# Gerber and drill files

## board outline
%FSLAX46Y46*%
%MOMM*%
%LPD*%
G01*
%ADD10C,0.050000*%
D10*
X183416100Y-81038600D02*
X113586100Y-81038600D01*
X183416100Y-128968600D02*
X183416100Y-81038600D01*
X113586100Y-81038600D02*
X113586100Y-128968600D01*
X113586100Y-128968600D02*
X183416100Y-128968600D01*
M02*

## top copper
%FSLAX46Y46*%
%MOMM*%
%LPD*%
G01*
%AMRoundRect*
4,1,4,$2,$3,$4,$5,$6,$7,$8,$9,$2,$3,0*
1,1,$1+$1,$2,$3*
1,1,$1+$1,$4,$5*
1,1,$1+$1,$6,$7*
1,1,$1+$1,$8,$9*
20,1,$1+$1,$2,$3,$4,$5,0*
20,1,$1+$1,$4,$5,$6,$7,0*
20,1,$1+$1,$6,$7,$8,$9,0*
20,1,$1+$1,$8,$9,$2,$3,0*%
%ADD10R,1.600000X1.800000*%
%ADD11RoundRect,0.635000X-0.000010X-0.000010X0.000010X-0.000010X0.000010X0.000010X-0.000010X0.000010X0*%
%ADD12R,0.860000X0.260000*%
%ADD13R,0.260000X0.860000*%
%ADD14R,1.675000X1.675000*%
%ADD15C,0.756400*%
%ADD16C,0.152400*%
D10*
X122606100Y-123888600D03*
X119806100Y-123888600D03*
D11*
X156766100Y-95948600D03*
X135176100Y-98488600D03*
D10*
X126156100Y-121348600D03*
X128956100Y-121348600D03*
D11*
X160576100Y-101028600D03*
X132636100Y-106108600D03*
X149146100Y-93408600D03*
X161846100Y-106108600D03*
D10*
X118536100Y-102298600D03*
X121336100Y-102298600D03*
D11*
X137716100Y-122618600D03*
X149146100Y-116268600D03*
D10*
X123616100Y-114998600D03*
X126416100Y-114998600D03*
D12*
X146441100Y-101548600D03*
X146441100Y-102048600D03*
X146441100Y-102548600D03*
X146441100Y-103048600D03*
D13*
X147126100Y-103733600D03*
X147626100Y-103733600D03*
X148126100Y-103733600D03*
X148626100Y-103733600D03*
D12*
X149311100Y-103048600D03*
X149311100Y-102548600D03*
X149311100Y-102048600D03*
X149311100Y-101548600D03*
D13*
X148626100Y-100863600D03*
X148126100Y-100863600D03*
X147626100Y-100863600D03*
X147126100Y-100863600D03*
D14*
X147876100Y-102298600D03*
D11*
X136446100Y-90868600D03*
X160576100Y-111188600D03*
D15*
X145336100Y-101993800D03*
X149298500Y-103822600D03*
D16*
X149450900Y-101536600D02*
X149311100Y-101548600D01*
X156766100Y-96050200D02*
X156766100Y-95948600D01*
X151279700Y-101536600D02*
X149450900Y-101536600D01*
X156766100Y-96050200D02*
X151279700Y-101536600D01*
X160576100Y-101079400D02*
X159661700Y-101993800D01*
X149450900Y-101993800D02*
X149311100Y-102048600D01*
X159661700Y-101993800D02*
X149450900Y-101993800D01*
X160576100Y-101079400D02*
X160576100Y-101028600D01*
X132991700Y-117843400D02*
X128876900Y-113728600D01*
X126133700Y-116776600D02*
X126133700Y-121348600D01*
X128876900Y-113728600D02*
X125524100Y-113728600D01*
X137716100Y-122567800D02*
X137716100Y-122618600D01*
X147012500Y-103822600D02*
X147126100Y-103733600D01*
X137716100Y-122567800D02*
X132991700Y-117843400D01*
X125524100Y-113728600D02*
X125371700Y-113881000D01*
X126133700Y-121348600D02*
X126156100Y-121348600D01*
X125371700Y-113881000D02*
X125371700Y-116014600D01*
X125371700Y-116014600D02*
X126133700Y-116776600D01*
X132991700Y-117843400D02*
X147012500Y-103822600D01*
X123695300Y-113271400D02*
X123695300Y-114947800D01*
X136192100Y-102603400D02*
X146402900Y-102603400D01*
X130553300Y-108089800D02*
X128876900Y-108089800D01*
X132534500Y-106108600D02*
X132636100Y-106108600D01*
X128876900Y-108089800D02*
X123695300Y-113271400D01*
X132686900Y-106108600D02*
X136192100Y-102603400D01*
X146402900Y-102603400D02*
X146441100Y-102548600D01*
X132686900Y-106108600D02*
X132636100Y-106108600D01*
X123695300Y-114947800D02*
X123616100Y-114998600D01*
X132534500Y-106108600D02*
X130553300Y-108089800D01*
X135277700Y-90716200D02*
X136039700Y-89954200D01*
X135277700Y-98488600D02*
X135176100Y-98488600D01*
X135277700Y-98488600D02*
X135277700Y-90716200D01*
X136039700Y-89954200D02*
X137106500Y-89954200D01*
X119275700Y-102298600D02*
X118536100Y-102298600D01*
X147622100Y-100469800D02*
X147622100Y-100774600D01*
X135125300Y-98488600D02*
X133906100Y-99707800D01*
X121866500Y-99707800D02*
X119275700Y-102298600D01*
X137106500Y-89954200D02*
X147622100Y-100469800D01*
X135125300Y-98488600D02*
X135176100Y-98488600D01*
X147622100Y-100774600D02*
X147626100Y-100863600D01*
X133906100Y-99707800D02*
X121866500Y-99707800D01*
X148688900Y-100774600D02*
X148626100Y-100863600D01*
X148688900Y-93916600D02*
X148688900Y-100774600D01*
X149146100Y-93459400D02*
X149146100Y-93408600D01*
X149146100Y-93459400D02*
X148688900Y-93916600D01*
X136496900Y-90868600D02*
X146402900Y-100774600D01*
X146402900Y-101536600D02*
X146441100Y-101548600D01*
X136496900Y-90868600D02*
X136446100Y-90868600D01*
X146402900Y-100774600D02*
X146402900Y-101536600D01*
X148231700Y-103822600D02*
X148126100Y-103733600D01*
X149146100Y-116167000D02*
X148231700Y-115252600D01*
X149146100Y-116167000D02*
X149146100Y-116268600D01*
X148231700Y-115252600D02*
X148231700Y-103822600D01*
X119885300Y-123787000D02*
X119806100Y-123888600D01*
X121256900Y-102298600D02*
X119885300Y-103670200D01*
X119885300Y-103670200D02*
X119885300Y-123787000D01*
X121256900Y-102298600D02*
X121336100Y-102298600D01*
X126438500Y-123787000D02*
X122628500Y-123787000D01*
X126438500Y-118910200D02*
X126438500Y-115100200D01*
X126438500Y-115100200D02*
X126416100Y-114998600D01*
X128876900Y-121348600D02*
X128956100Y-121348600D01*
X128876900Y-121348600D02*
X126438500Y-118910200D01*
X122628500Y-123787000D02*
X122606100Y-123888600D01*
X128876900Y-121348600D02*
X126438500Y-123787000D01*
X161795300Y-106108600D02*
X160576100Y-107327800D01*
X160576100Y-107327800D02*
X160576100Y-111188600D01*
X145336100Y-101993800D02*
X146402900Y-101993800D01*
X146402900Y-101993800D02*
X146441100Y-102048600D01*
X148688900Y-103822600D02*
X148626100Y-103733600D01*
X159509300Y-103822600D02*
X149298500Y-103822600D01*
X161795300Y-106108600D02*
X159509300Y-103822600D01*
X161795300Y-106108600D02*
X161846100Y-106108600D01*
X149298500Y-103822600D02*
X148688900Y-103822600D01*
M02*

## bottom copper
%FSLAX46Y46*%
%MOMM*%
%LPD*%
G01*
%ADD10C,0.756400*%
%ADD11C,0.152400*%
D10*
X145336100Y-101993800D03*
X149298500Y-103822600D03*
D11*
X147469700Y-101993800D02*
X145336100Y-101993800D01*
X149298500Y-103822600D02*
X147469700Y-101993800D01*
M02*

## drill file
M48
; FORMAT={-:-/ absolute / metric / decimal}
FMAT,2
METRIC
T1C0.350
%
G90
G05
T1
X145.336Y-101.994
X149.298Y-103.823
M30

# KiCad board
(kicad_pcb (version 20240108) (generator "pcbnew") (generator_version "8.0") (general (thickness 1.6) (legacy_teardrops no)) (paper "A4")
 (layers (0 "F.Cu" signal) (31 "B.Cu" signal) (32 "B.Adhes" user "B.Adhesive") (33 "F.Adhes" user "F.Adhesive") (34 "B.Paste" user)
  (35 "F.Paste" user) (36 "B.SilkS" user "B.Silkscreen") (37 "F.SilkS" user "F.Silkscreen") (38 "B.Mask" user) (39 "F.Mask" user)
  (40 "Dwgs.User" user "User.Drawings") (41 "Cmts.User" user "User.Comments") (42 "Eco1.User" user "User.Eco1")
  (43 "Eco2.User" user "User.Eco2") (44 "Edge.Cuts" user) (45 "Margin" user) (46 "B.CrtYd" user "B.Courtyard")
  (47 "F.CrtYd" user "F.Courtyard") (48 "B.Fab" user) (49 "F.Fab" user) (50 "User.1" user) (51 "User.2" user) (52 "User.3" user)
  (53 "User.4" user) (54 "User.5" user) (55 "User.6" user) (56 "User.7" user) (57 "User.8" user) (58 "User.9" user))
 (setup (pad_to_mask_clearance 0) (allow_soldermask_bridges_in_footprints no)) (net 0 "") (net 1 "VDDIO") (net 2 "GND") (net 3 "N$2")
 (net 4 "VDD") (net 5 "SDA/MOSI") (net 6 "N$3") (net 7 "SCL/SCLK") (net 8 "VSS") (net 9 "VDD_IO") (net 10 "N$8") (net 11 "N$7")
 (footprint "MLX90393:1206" (layer "F.Cu") (at 121.2061 123.8886 180)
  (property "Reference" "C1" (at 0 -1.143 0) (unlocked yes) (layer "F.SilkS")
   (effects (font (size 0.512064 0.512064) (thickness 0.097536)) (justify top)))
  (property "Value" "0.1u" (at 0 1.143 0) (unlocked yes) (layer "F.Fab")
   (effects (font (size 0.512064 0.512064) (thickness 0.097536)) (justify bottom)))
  (pad "1" smd rect (at -1.4 0 180) (size 1.6 1.8) (layers "F.Cu" "F.Paste" "F.Mask") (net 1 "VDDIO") (solder_mask_margin 0.1016)
   (thermal_bridge_angle 0))
  (pad "2" smd rect (at 1.4 0 180) (size 1.6 1.8) (layers "F.Cu" "F.Paste" "F.Mask") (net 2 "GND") (solder_mask_margin 0.1016)
   (thermal_bridge_angle 0)))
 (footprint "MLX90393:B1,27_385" (layer "F.Cu") (at 156.7661 95.9486)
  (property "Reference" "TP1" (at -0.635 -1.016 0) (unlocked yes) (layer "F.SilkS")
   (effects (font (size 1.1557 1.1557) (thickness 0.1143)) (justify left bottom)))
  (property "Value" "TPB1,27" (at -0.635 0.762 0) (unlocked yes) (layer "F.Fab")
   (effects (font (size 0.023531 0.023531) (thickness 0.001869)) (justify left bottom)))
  (pad "TP" smd roundrect (at 0 0) (size 1.27 1.27) (layers "F.Cu" "F.Mask") (roundrect_rratio 0.5) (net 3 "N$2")
   (solder_mask_margin 0.1016) (thermal_bridge_angle 0)))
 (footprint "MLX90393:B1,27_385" (layer "F.Cu") (at 135.1761 98.4886)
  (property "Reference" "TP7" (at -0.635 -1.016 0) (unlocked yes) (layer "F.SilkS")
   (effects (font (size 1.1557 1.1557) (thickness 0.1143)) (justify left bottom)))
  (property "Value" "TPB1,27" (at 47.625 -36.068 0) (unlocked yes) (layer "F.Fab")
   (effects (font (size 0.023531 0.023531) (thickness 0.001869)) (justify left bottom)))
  (pad "TP" smd roundrect (at 0 0) (size 1.27 1.27) (layers "F.Cu" "F.Mask") (roundrect_rratio 0.5) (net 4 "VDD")
   (solder_mask_margin 0.1016) (thermal_bridge_angle 0)))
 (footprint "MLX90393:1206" (layer "F.Cu") (at 127.5561 121.3486)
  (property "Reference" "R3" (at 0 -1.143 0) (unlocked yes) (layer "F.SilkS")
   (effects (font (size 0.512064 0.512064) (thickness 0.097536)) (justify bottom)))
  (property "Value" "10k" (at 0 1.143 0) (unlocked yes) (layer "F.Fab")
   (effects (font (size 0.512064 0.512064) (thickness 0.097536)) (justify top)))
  (pad "1" smd rect (at -1.4 0) (size 1.6 1.8) (layers "F.Cu" "F.Paste" "F.Mask") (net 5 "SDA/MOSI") (solder_mask_margin 0.1016)
   (thermal_bridge_angle 0))
  (pad "2" smd rect (at 1.4 0) (size 1.6 1.8) (layers "F.Cu" "F.Paste" "F.Mask") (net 1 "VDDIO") (solder_mask_margin 0.1016)
   (thermal_bridge_angle 0)))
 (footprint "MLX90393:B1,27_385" (layer "F.Cu") (at 160.5761 101.0286)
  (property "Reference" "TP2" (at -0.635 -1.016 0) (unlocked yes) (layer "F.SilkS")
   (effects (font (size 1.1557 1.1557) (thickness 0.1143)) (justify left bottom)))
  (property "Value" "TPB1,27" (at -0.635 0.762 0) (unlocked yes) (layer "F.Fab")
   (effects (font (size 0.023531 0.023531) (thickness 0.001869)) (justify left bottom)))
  (pad "TP" smd roundrect (at 0 0) (size 1.27 1.27) (layers "F.Cu" "F.Mask") (roundrect_rratio 0.5) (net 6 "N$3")
   (solder_mask_margin 0.1016) (thermal_bridge_angle 0)))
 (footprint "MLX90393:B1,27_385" (layer "F.Cu") (at 132.6361 106.1086)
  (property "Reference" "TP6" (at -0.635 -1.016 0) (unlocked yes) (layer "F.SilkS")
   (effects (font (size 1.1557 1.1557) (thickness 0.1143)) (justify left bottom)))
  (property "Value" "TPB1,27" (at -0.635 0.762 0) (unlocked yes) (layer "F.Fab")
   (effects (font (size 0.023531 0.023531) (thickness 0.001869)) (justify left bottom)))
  (pad "TP" smd roundrect (at 0 0) (size 1.27 1.27) (layers "F.Cu" "F.Mask") (roundrect_rratio 0.5) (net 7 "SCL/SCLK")
   (solder_mask_margin 0.1016) (thermal_bridge_angle 0)))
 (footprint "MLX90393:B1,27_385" (layer "F.Cu") (at 149.1461 93.4086)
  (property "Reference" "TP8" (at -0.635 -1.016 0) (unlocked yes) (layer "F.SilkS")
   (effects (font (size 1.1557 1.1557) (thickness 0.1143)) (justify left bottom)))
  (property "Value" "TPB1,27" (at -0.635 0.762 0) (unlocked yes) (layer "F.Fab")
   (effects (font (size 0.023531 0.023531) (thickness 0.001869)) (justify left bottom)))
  (pad "TP" smd roundrect (at 0 0) (size 1.27 1.27) (layers "F.Cu" "F.Mask") (roundrect_rratio 0.5) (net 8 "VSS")
   (solder_mask_margin 0.1016) (thermal_bridge_angle 0)))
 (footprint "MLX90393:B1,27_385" (layer "F.Cu") (at 161.8461 106.1086)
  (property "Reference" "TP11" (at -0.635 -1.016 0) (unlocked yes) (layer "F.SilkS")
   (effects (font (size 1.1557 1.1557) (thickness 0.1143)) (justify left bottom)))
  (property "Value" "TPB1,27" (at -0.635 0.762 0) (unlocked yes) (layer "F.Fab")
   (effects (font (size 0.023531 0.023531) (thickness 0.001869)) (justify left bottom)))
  (pad "TP" smd roundrect (at 0 0) (size 1.27 1.27) (layers "F.Cu" "F.Mask") (roundrect_rratio 0.5) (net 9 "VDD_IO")
   (solder_mask_margin 0.1016) (thermal_bridge_angle 0)))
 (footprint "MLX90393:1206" (layer "F.Cu") (at 119.9361 102.2986)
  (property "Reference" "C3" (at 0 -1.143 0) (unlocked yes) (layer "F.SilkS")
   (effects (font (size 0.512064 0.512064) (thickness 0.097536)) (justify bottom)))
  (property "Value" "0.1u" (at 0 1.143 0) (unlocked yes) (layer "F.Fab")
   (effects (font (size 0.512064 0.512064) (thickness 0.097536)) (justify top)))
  (pad "1" smd rect (at -1.4 0) (size 1.6 1.8) (layers "F.Cu" "F.Paste" "F.Mask") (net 4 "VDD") (solder_mask_margin 0.1016)
   (thermal_bridge_angle 0))
  (pad "2" smd rect (at 1.4 0) (size 1.6 1.8) (layers "F.Cu" "F.Paste" "F.Mask") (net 2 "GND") (solder_mask_margin 0.1016)
   (thermal_bridge_angle 0)))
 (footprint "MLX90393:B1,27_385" (layer "F.Cu") (at 137.7161 122.6186)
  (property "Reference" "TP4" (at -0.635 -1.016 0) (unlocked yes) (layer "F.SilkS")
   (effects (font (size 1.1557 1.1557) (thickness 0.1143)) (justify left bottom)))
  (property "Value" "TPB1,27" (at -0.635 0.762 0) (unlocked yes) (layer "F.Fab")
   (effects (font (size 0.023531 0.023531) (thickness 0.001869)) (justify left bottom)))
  (pad "TP" smd roundrect (at 0 0) (size 1.27 1.27) (layers "F.Cu" "F.Mask") (roundrect_rratio 0.5) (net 5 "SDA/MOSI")
   (solder_mask_margin 0.1016) (thermal_bridge_angle 0)))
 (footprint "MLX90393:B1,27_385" (layer "F.Cu") (at 149.1461 116.2686)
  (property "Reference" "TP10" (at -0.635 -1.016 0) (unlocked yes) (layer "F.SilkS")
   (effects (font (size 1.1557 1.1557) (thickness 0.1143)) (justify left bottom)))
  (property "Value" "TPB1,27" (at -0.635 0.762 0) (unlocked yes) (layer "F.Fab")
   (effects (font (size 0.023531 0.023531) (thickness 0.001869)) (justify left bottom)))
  (pad "TP" smd roundrect (at 0 0) (size 1.27 1.27) (layers "F.Cu" "F.Mask") (roundrect_rratio 0.5) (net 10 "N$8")
   (solder_mask_margin 0.1016) (thermal_bridge_angle 0)))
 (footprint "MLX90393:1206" (layer "F.Cu") (at 125.0161 114.9986)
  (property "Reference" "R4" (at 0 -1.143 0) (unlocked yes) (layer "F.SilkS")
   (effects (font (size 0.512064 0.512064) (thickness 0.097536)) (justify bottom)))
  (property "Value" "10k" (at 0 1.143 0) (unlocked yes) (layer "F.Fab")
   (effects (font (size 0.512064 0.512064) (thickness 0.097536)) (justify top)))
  (pad "1" smd rect (at -1.4 0) (size 1.6 1.8) (layers "F.Cu" "F.Paste" "F.Mask") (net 7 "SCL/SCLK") (solder_mask_margin 0.1016)
   (thermal_bridge_angle 0))
  (pad "2" smd rect (at 1.4 0) (size 1.6 1.8) (layers "F.Cu" "F.Paste" "F.Mask") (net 1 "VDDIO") (solder_mask_margin 0.1016)
   (thermal_bridge_angle 0)))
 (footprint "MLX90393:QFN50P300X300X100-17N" (layer "F.Cu") (at 147.8761 102.2986)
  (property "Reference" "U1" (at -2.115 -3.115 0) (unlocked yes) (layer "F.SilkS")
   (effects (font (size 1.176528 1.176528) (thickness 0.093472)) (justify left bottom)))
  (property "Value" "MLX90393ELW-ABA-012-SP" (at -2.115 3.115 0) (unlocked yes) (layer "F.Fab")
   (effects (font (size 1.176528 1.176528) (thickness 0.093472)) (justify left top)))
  (pad "1" smd rect (at -1.435 -0.75) (size 0.86 0.26) (layers "F.Cu" "F.Paste" "F.Mask") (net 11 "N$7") (solder_mask_margin 0.1016)
   (thermal_bridge_angle 0))
  (pad "2" smd rect (at -1.435 -0.25) (size 0.86 0.26) (layers "F.Cu" "F.Paste" "F.Mask") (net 9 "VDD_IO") (solder_mask_margin 0.1016)
   (thermal_bridge_angle 0))
  (pad "3" smd rect (at -1.435 0.25) (size 0.86 0.26) (layers "F.Cu" "F.Paste" "F.Mask") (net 7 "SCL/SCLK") (solder_mask_margin 0.1016)
   (thermal_bridge_angle 0))
  (pad "4" smd rect (at -1.435 0.75) (size 0.86 0.26) (layers "F.Cu" "F.Paste" "F.Mask") (solder_mask_margin 0.1016)
   (thermal_bridge_angle 0))
  (pad "5" smd rect (at -0.75 1.435) (size 0.26 0.86) (layers "F.Cu" "F.Paste" "F.Mask") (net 5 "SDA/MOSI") (solder_mask_margin 0.1016)
   (thermal_bridge_angle 0))
  (pad "6" smd rect (at -0.25 1.435) (size 0.26 0.86) (layers "F.Cu" "F.Paste" "F.Mask") (solder_mask_margin 0.1016)
   (thermal_bridge_angle 0))
  (pad "7" smd rect (at 0.25 1.435) (size 0.26 0.86) (layers "F.Cu" "F.Paste" "F.Mask") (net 10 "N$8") (solder_mask_margin 0.1016)
   (thermal_bridge_angle 0))
  (pad "8" smd rect (at 0.75 1.435) (size 0.26 0.86) (layers "F.Cu" "F.Paste" "F.Mask") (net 9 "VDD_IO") (solder_mask_margin 0.1016)
   (thermal_bridge_angle 0))
  (pad "9" smd rect (at 1.435 0.75) (size 0.86 0.26) (layers "F.Cu" "F.Paste" "F.Mask") (solder_mask_margin 0.1016) (thermal_bridge_angle 0))
  (pad "10" smd rect (at 1.435 0.25) (size 0.86 0.26) (layers "F.Cu" "F.Paste" "F.Mask") (solder_mask_margin 0.1016)
   (thermal_bridge_angle 0))
  (pad "11" smd rect (at 1.435 -0.25) (size 0.86 0.26) (layers "F.Cu" "F.Paste" "F.Mask") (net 6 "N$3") (solder_mask_margin 0.1016)
   (thermal_bridge_angle 0))
  (pad "12" smd rect (at 1.435 -0.75) (size 0.86 0.26) (layers "F.Cu" "F.Paste" "F.Mask") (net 3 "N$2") (solder_mask_margin 0.1016)
   (thermal_bridge_angle 0))
  (pad "13" smd rect (at 0.75 -1.435) (size 0.26 0.86) (layers "F.Cu" "F.Paste" "F.Mask") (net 8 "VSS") (solder_mask_margin 0.1016)
   (thermal_bridge_angle 0))
  (pad "14" smd rect (at 0.25 -1.435) (size 0.26 0.86) (layers "F.Cu" "F.Paste" "F.Mask") (solder_mask_margin 0.1016)
   (thermal_bridge_angle 0))
  (pad "15" smd rect (at -0.25 -1.435) (size 0.26 0.86) (layers "F.Cu" "F.Paste" "F.Mask") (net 4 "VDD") (solder_mask_margin 0.1016)
   (thermal_bridge_angle 0))
  (pad "16" smd rect (at -0.75 -1.435) (size 0.26 0.86) (layers "F.Cu" "F.Paste" "F.Mask") (solder_mask_margin 0.1016)
   (thermal_bridge_angle 0))
  (pad "17" smd rect (at 0 0) (size 1.675 1.675) (layers "F.Cu" "F.Mask") (solder_mask_margin 0.1016) (thermal_bridge_angle 0)))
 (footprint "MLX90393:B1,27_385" (layer "F.Cu") (at 136.4461 90.8686)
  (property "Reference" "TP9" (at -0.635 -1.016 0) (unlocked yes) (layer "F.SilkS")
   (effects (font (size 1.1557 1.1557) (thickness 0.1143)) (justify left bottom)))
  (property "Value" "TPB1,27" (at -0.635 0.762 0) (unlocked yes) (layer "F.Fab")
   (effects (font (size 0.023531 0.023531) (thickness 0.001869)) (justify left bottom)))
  (pad "TP" smd roundrect (at 0 0) (size 1.27 1.27) (layers "F.Cu" "F.Mask") (roundrect_rratio 0.5) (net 11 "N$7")
   (solder_mask_margin 0.1016) (thermal_bridge_angle 0)))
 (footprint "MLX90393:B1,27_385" (layer "F.Cu") (at 160.5761 111.1886)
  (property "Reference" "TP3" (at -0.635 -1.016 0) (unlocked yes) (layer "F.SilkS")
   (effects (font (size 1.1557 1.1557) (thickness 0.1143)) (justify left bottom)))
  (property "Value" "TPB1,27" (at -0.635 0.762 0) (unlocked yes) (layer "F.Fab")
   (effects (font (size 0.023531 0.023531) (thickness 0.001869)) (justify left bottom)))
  (pad "TP" smd roundrect (at 0 0) (size 1.27 1.27) (layers "F.Cu" "F.Mask") (roundrect_rratio 0.5) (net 9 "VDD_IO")
   (solder_mask_margin 0.1016) (thermal_bridge_angle 0)))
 (gr_line (start 183.4161 81.0386) (end 113.5861 81.0386) (stroke (width 0.05) (type solid)) (layer "Edge.Cuts"))
 (gr_line (start 183.4161 128.9686) (end 183.4161 81.0386) (stroke (width 0.05) (type solid)) (layer "Edge.Cuts"))
 (gr_line (start 113.5861 81.0386) (end 113.5861 128.9686) (stroke (width 0.05) (type solid)) (layer "Edge.Cuts"))
 (gr_line (start 113.5861 128.9686) (end 183.4161 128.9686) (stroke (width 0.05) (type solid)) (layer "Edge.Cuts"))
 (segment (start 149.4509 101.5366) (end 149.3111 101.5486) (width 0.1524) (layer "F.Cu") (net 3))
 (segment (start 156.7661 96.0502) (end 156.7661 95.9486) (width 0.1524) (layer "F.Cu") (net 3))
 (segment (start 151.2797 101.5366) (end 149.4509 101.5366) (width 0.1524) (layer "F.Cu") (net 3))
 (segment (start 156.7661 96.0502) (end 151.2797 101.5366) (width 0.1524) (layer "F.Cu") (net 3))
 (segment (start 160.5761 101.0794) (end 159.6617 101.9938) (width 0.1524) (layer "F.Cu") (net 6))
 (segment (start 149.4509 101.9938) (end 149.3111 102.0486) (width 0.1524) (layer "F.Cu") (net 6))
 (segment (start 159.6617 101.9938) (end 149.4509 101.9938) (width 0.1524) (layer "F.Cu") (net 6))
 (segment (start 160.5761 101.0794) (end 160.5761 101.0286) (width 0.1524) (layer "F.Cu") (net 6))
 (segment (start 132.9917 117.8434) (end 128.8769 113.7286) (width 0.1524) (layer "F.Cu") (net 5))
 (segment (start 126.1337 116.7766) (end 126.1337 121.3486) (width 0.1524) (layer "F.Cu") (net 5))
 (segment (start 128.8769 113.7286) (end 125.5241 113.7286) (width 0.1524) (layer "F.Cu") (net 5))
 (segment (start 137.7161 122.5678) (end 137.7161 122.6186) (width 0.1524) (layer "F.Cu") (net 5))
 (segment (start 147.0125 103.8226) (end 147.1261 103.7336) (width 0.1524) (layer "F.Cu") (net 5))
 (segment (start 137.7161 122.5678) (end 132.9917 117.8434) (width 0.1524) (layer "F.Cu") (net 5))
 (segment (start 125.5241 113.7286) (end 125.3717 113.881) (width 0.1524) (layer "F.Cu") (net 5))
 (segment (start 126.1337 121.3486) (end 126.1561 121.3486) (width 0.1524) (layer "F.Cu") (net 5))
 (segment (start 125.3717 113.881) (end 125.3717 116.0146) (width 0.1524) (layer "F.Cu") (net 5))
 (segment (start 125.3717 116.0146) (end 126.1337 116.7766) (width 0.1524) (layer "F.Cu") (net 5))
 (segment (start 132.9917 117.8434) (end 147.0125 103.8226) (width 0.1524) (layer "F.Cu") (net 5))
 (segment (start 123.6953 113.2714) (end 123.6953 114.9478) (width 0.1524) (layer "F.Cu") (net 7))
 (segment (start 136.1921 102.6034) (end 146.4029 102.6034) (width 0.1524) (layer "F.Cu") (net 7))
 (segment (start 130.5533 108.0898) (end 128.8769 108.0898) (width 0.1524) (layer "F.Cu") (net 7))
 (segment (start 132.5345 106.1086) (end 132.6361 106.1086) (width 0.1524) (layer "F.Cu") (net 7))
 (segment (start 128.8769 108.0898) (end 123.6953 113.2714) (width 0.1524) (layer "F.Cu") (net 7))
 (segment (start 132.6869 106.1086) (end 136.1921 102.6034) (width 0.1524) (layer "F.Cu") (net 7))
 (segment (start 146.4029 102.6034) (end 146.4411 102.5486) (width 0.1524) (layer "F.Cu") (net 7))
 (segment (start 132.6869 106.1086) (end 132.6361 106.1086) (width 0.1524) (layer "F.Cu") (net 7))
 (segment (start 123.6953 114.9478) (end 123.6161 114.9986) (width 0.1524) (layer "F.Cu") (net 7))
 (segment (start 132.5345 106.1086) (end 130.5533 108.0898) (width 0.1524) (layer "F.Cu") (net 7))
 (segment (start 135.2777 90.7162) (end 136.0397 89.9542) (width 0.1524) (layer "F.Cu") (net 4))
 (segment (start 135.2777 98.4886) (end 135.1761 98.4886) (width 0.1524) (layer "F.Cu") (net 4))
 (segment (start 135.2777 98.4886) (end 135.2777 90.7162) (width 0.1524) (layer "F.Cu") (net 4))
 (segment (start 136.0397 89.9542) (end 137.1065 89.9542) (width 0.1524) (layer "F.Cu") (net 4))
 (segment (start 119.2757 102.2986) (end 118.5361 102.2986) (width 0.1524) (layer "F.Cu") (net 4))
 (segment (start 147.6221 100.4698) (end 147.6221 100.7746) (width 0.1524) (layer "F.Cu") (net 4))
 (segment (start 135.1253 98.4886) (end 133.9061 99.7078) (width 0.1524) (layer "F.Cu") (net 4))
 (segment (start 121.8665 99.7078) (end 119.2757 102.2986) (width 0.1524) (layer "F.Cu") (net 4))
 (segment (start 137.1065 89.9542) (end 147.6221 100.4698) (width 0.1524) (layer "F.Cu") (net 4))
 (segment (start 135.1253 98.4886) (end 135.1761 98.4886) (width 0.1524) (layer "F.Cu") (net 4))
 (segment (start 147.6221 100.7746) (end 147.6261 100.8636) (width 0.1524) (layer "F.Cu") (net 4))
 (segment (start 133.9061 99.7078) (end 121.8665 99.7078) (width 0.1524) (layer "F.Cu") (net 4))
 (segment (start 148.6889 100.7746) (end 148.6261 100.8636) (width 0.1524) (layer "F.Cu") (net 8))
 (segment (start 148.6889 93.9166) (end 148.6889 100.7746) (width 0.1524) (layer "F.Cu") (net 8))
 (segment (start 149.1461 93.4594) (end 149.1461 93.4086) (width 0.1524) (layer "F.Cu") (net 8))
 (segment (start 149.1461 93.4594) (end 148.6889 93.9166) (width 0.1524) (layer "F.Cu") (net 8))
 (segment (start 136.4969 90.8686) (end 146.4029 100.7746) (width 0.1524) (layer "F.Cu") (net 11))
 (segment (start 146.4029 101.5366) (end 146.4411 101.5486) (width 0.1524) (layer "F.Cu") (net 11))
 (segment (start 136.4969 90.8686) (end 136.4461 90.8686) (width 0.1524) (layer "F.Cu") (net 11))
 (segment (start 146.4029 100.7746) (end 146.4029 101.5366) (width 0.1524) (layer "F.Cu") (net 11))
 (segment (start 148.2317 103.8226) (end 148.1261 103.7336) (width 0.1524) (layer "F.Cu") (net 10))
 (segment (start 149.1461 116.167) (end 148.2317 115.2526) (width 0.1524) (layer "F.Cu") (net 10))
 (segment (start 149.1461 116.167) (end 149.1461 116.2686) (width 0.1524) (layer "F.Cu") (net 10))
 (segment (start 148.2317 115.2526) (end 148.2317 103.8226) (width 0.1524) (layer "F.Cu") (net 10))
 (segment (start 119.8853 123.787) (end 119.8061 123.8886) (width 0.1524) (layer "F.Cu") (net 2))
 (segment (start 121.2569 102.2986) (end 119.8853 103.6702) (width 0.1524) (layer "F.Cu") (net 2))
 (segment (start 119.8853 103.6702) (end 119.8853 123.787) (width 0.1524) (layer "F.Cu") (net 2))
 (segment (start 121.2569 102.2986) (end 121.3361 102.2986) (width 0.1524) (layer "F.Cu") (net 2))
 (segment (start 126.4385 123.787) (end 122.6285 123.787) (width 0.1524) (layer "F.Cu") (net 1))
 (segment (start 126.4385 118.9102) (end 126.4385 115.1002) (width 0.1524) (layer "F.Cu") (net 1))
 (segment (start 126.4385 115.1002) (end 126.4161 114.9986) (width 0.1524) (layer "F.Cu") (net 1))
 (segment (start 128.8769 121.3486) (end 128.9561 121.3486) (width 0.1524) (layer "F.Cu") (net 1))
 (segment (start 128.8769 121.3486) (end 126.4385 118.9102) (width 0.1524) (layer "F.Cu") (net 1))
 (segment (start 122.6285 123.787) (end 122.6061 123.8886) (width 0.1524) (layer "F.Cu") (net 1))
 (segment (start 128.8769 121.3486) (end 126.4385 123.787) (width 0.1524) (layer "F.Cu") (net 1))
 (segment (start 161.7953 106.1086) (end 160.5761 107.3278) (width 0.1524) (layer "F.Cu") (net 9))
 (segment (start 160.5761 107.3278) (end 160.5761 111.1886) (width 0.1524) (layer "F.Cu") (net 9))
 (segment (start 145.3361 101.9938) (end 146.4029 101.9938) (width 0.1524) (layer "F.Cu") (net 9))
 (segment (start 146.4029 101.9938) (end 146.4411 102.0486) (width 0.1524) (layer "F.Cu") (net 9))
 (segment (start 148.6889 103.8226) (end 148.6261 103.7336) (width 0.1524) (layer "F.Cu") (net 9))
 (segment (start 159.5093 103.8226) (end 149.2985 103.8226) (width 0.1524) (layer "F.Cu") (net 9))
 (segment (start 161.7953 106.1086) (end 159.5093 103.8226) (width 0.1524) (layer "F.Cu") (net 9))
 (segment (start 161.7953 106.1086) (end 161.8461 106.1086) (width 0.1524) (layer "F.Cu") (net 9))
 (segment (start 149.2985 103.8226) (end 148.6889 103.8226) (width 0.1524) (layer "F.Cu") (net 9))
 (via (at 145.3361 101.9938) (size 0.7564) (drill 0.35) (layers "F.Cu" "B.Cu") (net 9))
 (via (at 149.2985 103.8226) (size 0.7564) (drill 0.35) (layers "F.Cu" "B.Cu") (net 9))
 (segment (start 147.4697 101.9938) (end 145.3361 101.9938) (width 0.1524) (layer "B.Cu") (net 9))
 (segment (start 149.2985 103.8226) (end 147.4697 101.9938) (width 0.1524) (layer "B.Cu") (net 9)))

